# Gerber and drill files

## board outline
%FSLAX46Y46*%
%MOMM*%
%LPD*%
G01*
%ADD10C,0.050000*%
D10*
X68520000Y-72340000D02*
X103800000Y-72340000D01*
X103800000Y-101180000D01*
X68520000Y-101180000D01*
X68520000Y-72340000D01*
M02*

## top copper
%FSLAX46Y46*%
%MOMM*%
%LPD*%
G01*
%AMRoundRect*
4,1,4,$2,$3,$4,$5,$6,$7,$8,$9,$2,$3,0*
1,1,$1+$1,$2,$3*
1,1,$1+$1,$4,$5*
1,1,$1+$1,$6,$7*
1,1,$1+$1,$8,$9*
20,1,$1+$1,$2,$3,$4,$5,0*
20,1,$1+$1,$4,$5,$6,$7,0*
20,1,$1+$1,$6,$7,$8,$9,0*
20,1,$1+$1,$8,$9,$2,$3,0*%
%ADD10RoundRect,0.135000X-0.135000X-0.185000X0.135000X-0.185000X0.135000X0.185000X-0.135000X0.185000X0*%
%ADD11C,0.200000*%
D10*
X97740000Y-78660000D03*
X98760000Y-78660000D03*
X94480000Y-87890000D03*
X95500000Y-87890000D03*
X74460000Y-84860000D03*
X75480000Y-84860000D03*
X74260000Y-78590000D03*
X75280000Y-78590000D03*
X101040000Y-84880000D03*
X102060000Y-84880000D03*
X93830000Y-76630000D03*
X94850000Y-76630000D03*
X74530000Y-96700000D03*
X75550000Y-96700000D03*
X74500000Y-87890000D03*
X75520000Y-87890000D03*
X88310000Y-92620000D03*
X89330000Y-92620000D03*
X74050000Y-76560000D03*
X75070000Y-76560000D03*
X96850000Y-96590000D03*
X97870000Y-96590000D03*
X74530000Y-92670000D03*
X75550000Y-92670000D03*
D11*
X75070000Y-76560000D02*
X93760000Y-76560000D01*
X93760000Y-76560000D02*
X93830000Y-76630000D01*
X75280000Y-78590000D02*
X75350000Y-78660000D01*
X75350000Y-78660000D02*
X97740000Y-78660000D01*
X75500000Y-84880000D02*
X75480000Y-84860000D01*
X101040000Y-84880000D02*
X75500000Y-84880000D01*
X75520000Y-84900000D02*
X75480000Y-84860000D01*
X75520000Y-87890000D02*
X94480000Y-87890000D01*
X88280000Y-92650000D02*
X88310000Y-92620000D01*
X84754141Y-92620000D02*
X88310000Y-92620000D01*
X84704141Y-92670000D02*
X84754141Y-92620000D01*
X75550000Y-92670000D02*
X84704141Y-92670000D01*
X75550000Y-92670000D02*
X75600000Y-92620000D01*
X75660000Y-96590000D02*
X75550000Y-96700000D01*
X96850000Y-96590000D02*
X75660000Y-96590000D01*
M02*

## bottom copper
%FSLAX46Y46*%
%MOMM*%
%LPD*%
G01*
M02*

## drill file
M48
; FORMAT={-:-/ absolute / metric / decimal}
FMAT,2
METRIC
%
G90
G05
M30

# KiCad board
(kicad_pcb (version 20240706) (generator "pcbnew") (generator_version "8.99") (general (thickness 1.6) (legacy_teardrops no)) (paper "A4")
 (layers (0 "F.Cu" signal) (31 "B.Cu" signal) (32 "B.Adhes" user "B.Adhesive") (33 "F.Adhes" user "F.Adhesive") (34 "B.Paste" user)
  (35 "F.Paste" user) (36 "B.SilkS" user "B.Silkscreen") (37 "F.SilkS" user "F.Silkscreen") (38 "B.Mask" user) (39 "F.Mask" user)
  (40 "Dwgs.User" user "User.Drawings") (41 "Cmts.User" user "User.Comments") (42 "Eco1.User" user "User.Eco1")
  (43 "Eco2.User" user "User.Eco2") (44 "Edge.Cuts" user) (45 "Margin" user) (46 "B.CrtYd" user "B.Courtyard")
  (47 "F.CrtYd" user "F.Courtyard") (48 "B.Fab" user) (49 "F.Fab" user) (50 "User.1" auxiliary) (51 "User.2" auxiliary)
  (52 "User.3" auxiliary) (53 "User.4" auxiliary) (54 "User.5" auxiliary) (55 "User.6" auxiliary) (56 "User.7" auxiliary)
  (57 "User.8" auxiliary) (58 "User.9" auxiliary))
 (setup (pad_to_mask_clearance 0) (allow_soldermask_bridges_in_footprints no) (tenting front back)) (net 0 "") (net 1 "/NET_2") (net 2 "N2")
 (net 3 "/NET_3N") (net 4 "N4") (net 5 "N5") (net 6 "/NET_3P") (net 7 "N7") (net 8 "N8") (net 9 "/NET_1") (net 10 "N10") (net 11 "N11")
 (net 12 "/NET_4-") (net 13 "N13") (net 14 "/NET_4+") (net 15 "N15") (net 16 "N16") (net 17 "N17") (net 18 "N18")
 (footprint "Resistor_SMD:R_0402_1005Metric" (layer "F.Cu") (at 98.25 78.66)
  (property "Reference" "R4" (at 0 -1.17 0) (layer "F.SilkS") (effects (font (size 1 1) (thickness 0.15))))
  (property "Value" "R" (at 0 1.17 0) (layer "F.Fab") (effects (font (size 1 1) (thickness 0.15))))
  (pad "1" smd roundrect (at -0.51 0) (size 0.54 0.64) (layers "F.Cu" "F.Paste" "F.Mask") (roundrect_rratio 0.25) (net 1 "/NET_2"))
  (pad "2" smd roundrect (at 0.51 0) (size 0.54 0.64) (layers "F.Cu" "F.Paste" "F.Mask") (roundrect_rratio 0.25) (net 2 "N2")))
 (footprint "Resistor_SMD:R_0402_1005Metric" (layer "F.Cu") (at 94.99 87.89)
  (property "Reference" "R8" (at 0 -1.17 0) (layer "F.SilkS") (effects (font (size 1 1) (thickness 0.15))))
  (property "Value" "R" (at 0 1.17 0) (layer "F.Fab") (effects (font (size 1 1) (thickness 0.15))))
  (pad "1" smd roundrect (at -0.51 0) (size 0.54 0.64) (layers "F.Cu" "F.Paste" "F.Mask") (roundrect_rratio 0.25) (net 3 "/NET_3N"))
  (pad "2" smd roundrect (at 0.51 0) (size 0.54 0.64) (layers "F.Cu" "F.Paste" "F.Mask") (roundrect_rratio 0.25) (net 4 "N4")))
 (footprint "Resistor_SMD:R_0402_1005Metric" (layer "F.Cu") (at 74.97 84.86)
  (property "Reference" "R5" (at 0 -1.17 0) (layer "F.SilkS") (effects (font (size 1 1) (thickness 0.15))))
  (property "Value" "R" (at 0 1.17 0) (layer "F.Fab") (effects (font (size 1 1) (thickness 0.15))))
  (pad "1" smd roundrect (at -0.51 0) (size 0.54 0.64) (layers "F.Cu" "F.Paste" "F.Mask") (roundrect_rratio 0.25) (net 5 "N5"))
  (pad "2" smd roundrect (at 0.51 0) (size 0.54 0.64) (layers "F.Cu" "F.Paste" "F.Mask") (roundrect_rratio 0.25) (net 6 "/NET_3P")))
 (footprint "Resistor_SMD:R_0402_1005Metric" (layer "F.Cu") (at 74.77 78.59)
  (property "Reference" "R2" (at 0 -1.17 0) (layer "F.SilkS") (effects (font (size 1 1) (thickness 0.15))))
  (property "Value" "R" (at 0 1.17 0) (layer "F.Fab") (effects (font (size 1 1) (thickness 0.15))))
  (pad "1" smd roundrect (at -0.51 0) (size 0.54 0.64) (layers "F.Cu" "F.Paste" "F.Mask") (roundrect_rratio 0.25) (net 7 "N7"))
  (pad "2" smd roundrect (at 0.51 0) (size 0.54 0.64) (layers "F.Cu" "F.Paste" "F.Mask") (roundrect_rratio 0.25) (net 1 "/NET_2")))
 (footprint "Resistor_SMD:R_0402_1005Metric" (layer "F.Cu") (at 101.55 84.88)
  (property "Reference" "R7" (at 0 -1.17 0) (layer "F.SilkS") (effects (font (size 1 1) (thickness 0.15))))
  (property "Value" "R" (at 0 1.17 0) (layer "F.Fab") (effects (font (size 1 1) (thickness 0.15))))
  (pad "1" smd roundrect (at -0.51 0) (size 0.54 0.64) (layers "F.Cu" "F.Paste" "F.Mask") (roundrect_rratio 0.25) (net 6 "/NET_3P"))
  (pad "2" smd roundrect (at 0.51 0) (size 0.54 0.64) (layers "F.Cu" "F.Paste" "F.Mask") (roundrect_rratio 0.25) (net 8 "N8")))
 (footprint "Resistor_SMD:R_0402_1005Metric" (layer "F.Cu") (at 94.34 76.63)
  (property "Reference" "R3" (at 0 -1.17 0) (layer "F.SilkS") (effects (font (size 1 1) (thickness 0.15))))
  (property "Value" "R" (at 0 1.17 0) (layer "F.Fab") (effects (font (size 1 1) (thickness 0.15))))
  (pad "1" smd roundrect (at -0.51 0) (size 0.54 0.64) (layers "F.Cu" "F.Paste" "F.Mask") (roundrect_rratio 0.25) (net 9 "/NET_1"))
  (pad "2" smd roundrect (at 0.51 0) (size 0.54 0.64) (layers "F.Cu" "F.Paste" "F.Mask") (roundrect_rratio 0.25) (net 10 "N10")))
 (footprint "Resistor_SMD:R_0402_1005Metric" (layer "F.Cu") (at 75.04 96.7)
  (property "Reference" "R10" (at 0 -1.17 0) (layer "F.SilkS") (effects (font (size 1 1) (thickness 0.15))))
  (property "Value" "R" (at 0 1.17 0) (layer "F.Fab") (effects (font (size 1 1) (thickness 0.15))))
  (pad "1" smd roundrect (at -0.51 0) (size 0.54 0.64) (layers "F.Cu" "F.Paste" "F.Mask") (roundrect_rratio 0.25) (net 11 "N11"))
  (pad "2" smd roundrect (at 0.51 0) (size 0.54 0.64) (layers "F.Cu" "F.Paste" "F.Mask") (roundrect_rratio 0.25) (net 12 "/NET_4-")))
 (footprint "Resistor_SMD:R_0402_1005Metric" (layer "F.Cu") (at 75.01 87.89)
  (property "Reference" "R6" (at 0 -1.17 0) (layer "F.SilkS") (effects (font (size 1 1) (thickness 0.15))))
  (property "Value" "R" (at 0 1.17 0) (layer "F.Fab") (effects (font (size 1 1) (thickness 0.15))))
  (pad "1" smd roundrect (at -0.51 0) (size 0.54 0.64) (layers "F.Cu" "F.Paste" "F.Mask") (roundrect_rratio 0.25) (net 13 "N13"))
  (pad "2" smd roundrect (at 0.51 0) (size 0.54 0.64) (layers "F.Cu" "F.Paste" "F.Mask") (roundrect_rratio 0.25) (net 3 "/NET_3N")))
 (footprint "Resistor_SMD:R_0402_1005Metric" (layer "F.Cu") (at 88.82 92.62)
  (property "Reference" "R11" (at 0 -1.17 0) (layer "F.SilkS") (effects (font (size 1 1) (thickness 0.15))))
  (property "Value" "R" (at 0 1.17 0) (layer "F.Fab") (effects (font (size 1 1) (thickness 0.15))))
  (pad "1" smd roundrect (at -0.51 0) (size 0.54 0.64) (layers "F.Cu" "F.Paste" "F.Mask") (roundrect_rratio 0.25) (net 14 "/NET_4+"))
  (pad "2" smd roundrect (at 0.51 0) (size 0.54 0.64) (layers "F.Cu" "F.Paste" "F.Mask") (roundrect_rratio 0.25) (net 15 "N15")))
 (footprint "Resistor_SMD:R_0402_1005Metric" (layer "F.Cu") (at 74.56 76.56)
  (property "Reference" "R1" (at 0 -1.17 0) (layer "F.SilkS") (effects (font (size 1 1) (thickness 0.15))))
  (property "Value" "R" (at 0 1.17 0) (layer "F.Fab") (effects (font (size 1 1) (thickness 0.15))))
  (pad "1" smd roundrect (at -0.51 0) (size 0.54 0.64) (layers "F.Cu" "F.Paste" "F.Mask") (roundrect_rratio 0.25) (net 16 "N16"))
  (pad "2" smd roundrect (at 0.51 0) (size 0.54 0.64) (layers "F.Cu" "F.Paste" "F.Mask") (roundrect_rratio 0.25) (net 9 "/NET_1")))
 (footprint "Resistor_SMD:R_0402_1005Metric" (layer "F.Cu") (at 97.36 96.59)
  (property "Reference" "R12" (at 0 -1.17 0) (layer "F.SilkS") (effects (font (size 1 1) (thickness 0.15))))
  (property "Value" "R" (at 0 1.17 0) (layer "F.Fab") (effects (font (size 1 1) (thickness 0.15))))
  (pad "1" smd roundrect (at -0.51 0) (size 0.54 0.64) (layers "F.Cu" "F.Paste" "F.Mask") (roundrect_rratio 0.25) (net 12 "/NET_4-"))
  (pad "2" smd roundrect (at 0.51 0) (size 0.54 0.64) (layers "F.Cu" "F.Paste" "F.Mask") (roundrect_rratio 0.25) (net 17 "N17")))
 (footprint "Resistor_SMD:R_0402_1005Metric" (layer "F.Cu") (at 75.04 92.67)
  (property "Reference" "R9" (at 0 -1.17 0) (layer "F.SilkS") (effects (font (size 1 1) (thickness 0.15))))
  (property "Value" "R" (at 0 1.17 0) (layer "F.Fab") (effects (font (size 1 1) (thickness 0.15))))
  (pad "1" smd roundrect (at -0.51 0) (size 0.54 0.64) (layers "F.Cu" "F.Paste" "F.Mask") (roundrect_rratio 0.25) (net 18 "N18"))
  (pad "2" smd roundrect (at 0.51 0) (size 0.54 0.64) (layers "F.Cu" "F.Paste" "F.Mask") (roundrect_rratio 0.25) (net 14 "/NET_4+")))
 (gr_rect (start 68.52 72.34) (end 103.8 101.18) (stroke (width 0.05) (type default)) (fill none) (layer "Edge.Cuts"))
 (segment (start 75.07 76.56) (end 93.76 76.56) (width 0.2) (layer "F.Cu") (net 9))
 (segment (start 93.76 76.56) (end 93.83 76.63) (width 0.2) (layer "F.Cu") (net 9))
 (segment (start 75.28 78.59) (end 75.35 78.66) (width 0.2) (layer "F.Cu") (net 1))
 (segment (start 75.35 78.66) (end 97.74 78.66) (width 0.2) (layer "F.Cu") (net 1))
 (segment (start 75.5 84.88) (end 75.48 84.86) (width 0.2) (layer "F.Cu") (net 6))
 (segment (start 101.04 84.88) (end 75.5 84.88) (width 0.2) (layer "F.Cu") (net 6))
 (segment (start 75.52 84.9) (end 75.48 84.86) (width 0.2) (layer "F.Cu") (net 6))
 (segment (start 75.52 87.89) (end 94.48 87.89) (width 0.2) (layer "F.Cu") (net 3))
 (segment (start 88.28 92.65) (end 88.31 92.62) (width 0.2) (layer "F.Cu") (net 14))
 (segment (start 84.754141 92.62) (end 88.31 92.62) (width 0.2) (layer "F.Cu") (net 14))
 (segment (start 84.704141 92.67) (end 84.754141 92.62) (width 0.2) (layer "F.Cu") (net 14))
 (segment (start 75.55 92.67) (end 84.704141 92.67) (width 0.2) (layer "F.Cu") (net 14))
 (segment (start 75.55 92.67) (end 75.6 92.62) (width 0.2) (layer "F.Cu") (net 14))
 (segment (start 75.66 96.59) (end 75.55 96.7) (width 0.2) (layer "F.Cu") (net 12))
 (segment (start 96.85 96.59) (end 75.66 96.59) (width 0.2) (layer "F.Cu") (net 12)))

